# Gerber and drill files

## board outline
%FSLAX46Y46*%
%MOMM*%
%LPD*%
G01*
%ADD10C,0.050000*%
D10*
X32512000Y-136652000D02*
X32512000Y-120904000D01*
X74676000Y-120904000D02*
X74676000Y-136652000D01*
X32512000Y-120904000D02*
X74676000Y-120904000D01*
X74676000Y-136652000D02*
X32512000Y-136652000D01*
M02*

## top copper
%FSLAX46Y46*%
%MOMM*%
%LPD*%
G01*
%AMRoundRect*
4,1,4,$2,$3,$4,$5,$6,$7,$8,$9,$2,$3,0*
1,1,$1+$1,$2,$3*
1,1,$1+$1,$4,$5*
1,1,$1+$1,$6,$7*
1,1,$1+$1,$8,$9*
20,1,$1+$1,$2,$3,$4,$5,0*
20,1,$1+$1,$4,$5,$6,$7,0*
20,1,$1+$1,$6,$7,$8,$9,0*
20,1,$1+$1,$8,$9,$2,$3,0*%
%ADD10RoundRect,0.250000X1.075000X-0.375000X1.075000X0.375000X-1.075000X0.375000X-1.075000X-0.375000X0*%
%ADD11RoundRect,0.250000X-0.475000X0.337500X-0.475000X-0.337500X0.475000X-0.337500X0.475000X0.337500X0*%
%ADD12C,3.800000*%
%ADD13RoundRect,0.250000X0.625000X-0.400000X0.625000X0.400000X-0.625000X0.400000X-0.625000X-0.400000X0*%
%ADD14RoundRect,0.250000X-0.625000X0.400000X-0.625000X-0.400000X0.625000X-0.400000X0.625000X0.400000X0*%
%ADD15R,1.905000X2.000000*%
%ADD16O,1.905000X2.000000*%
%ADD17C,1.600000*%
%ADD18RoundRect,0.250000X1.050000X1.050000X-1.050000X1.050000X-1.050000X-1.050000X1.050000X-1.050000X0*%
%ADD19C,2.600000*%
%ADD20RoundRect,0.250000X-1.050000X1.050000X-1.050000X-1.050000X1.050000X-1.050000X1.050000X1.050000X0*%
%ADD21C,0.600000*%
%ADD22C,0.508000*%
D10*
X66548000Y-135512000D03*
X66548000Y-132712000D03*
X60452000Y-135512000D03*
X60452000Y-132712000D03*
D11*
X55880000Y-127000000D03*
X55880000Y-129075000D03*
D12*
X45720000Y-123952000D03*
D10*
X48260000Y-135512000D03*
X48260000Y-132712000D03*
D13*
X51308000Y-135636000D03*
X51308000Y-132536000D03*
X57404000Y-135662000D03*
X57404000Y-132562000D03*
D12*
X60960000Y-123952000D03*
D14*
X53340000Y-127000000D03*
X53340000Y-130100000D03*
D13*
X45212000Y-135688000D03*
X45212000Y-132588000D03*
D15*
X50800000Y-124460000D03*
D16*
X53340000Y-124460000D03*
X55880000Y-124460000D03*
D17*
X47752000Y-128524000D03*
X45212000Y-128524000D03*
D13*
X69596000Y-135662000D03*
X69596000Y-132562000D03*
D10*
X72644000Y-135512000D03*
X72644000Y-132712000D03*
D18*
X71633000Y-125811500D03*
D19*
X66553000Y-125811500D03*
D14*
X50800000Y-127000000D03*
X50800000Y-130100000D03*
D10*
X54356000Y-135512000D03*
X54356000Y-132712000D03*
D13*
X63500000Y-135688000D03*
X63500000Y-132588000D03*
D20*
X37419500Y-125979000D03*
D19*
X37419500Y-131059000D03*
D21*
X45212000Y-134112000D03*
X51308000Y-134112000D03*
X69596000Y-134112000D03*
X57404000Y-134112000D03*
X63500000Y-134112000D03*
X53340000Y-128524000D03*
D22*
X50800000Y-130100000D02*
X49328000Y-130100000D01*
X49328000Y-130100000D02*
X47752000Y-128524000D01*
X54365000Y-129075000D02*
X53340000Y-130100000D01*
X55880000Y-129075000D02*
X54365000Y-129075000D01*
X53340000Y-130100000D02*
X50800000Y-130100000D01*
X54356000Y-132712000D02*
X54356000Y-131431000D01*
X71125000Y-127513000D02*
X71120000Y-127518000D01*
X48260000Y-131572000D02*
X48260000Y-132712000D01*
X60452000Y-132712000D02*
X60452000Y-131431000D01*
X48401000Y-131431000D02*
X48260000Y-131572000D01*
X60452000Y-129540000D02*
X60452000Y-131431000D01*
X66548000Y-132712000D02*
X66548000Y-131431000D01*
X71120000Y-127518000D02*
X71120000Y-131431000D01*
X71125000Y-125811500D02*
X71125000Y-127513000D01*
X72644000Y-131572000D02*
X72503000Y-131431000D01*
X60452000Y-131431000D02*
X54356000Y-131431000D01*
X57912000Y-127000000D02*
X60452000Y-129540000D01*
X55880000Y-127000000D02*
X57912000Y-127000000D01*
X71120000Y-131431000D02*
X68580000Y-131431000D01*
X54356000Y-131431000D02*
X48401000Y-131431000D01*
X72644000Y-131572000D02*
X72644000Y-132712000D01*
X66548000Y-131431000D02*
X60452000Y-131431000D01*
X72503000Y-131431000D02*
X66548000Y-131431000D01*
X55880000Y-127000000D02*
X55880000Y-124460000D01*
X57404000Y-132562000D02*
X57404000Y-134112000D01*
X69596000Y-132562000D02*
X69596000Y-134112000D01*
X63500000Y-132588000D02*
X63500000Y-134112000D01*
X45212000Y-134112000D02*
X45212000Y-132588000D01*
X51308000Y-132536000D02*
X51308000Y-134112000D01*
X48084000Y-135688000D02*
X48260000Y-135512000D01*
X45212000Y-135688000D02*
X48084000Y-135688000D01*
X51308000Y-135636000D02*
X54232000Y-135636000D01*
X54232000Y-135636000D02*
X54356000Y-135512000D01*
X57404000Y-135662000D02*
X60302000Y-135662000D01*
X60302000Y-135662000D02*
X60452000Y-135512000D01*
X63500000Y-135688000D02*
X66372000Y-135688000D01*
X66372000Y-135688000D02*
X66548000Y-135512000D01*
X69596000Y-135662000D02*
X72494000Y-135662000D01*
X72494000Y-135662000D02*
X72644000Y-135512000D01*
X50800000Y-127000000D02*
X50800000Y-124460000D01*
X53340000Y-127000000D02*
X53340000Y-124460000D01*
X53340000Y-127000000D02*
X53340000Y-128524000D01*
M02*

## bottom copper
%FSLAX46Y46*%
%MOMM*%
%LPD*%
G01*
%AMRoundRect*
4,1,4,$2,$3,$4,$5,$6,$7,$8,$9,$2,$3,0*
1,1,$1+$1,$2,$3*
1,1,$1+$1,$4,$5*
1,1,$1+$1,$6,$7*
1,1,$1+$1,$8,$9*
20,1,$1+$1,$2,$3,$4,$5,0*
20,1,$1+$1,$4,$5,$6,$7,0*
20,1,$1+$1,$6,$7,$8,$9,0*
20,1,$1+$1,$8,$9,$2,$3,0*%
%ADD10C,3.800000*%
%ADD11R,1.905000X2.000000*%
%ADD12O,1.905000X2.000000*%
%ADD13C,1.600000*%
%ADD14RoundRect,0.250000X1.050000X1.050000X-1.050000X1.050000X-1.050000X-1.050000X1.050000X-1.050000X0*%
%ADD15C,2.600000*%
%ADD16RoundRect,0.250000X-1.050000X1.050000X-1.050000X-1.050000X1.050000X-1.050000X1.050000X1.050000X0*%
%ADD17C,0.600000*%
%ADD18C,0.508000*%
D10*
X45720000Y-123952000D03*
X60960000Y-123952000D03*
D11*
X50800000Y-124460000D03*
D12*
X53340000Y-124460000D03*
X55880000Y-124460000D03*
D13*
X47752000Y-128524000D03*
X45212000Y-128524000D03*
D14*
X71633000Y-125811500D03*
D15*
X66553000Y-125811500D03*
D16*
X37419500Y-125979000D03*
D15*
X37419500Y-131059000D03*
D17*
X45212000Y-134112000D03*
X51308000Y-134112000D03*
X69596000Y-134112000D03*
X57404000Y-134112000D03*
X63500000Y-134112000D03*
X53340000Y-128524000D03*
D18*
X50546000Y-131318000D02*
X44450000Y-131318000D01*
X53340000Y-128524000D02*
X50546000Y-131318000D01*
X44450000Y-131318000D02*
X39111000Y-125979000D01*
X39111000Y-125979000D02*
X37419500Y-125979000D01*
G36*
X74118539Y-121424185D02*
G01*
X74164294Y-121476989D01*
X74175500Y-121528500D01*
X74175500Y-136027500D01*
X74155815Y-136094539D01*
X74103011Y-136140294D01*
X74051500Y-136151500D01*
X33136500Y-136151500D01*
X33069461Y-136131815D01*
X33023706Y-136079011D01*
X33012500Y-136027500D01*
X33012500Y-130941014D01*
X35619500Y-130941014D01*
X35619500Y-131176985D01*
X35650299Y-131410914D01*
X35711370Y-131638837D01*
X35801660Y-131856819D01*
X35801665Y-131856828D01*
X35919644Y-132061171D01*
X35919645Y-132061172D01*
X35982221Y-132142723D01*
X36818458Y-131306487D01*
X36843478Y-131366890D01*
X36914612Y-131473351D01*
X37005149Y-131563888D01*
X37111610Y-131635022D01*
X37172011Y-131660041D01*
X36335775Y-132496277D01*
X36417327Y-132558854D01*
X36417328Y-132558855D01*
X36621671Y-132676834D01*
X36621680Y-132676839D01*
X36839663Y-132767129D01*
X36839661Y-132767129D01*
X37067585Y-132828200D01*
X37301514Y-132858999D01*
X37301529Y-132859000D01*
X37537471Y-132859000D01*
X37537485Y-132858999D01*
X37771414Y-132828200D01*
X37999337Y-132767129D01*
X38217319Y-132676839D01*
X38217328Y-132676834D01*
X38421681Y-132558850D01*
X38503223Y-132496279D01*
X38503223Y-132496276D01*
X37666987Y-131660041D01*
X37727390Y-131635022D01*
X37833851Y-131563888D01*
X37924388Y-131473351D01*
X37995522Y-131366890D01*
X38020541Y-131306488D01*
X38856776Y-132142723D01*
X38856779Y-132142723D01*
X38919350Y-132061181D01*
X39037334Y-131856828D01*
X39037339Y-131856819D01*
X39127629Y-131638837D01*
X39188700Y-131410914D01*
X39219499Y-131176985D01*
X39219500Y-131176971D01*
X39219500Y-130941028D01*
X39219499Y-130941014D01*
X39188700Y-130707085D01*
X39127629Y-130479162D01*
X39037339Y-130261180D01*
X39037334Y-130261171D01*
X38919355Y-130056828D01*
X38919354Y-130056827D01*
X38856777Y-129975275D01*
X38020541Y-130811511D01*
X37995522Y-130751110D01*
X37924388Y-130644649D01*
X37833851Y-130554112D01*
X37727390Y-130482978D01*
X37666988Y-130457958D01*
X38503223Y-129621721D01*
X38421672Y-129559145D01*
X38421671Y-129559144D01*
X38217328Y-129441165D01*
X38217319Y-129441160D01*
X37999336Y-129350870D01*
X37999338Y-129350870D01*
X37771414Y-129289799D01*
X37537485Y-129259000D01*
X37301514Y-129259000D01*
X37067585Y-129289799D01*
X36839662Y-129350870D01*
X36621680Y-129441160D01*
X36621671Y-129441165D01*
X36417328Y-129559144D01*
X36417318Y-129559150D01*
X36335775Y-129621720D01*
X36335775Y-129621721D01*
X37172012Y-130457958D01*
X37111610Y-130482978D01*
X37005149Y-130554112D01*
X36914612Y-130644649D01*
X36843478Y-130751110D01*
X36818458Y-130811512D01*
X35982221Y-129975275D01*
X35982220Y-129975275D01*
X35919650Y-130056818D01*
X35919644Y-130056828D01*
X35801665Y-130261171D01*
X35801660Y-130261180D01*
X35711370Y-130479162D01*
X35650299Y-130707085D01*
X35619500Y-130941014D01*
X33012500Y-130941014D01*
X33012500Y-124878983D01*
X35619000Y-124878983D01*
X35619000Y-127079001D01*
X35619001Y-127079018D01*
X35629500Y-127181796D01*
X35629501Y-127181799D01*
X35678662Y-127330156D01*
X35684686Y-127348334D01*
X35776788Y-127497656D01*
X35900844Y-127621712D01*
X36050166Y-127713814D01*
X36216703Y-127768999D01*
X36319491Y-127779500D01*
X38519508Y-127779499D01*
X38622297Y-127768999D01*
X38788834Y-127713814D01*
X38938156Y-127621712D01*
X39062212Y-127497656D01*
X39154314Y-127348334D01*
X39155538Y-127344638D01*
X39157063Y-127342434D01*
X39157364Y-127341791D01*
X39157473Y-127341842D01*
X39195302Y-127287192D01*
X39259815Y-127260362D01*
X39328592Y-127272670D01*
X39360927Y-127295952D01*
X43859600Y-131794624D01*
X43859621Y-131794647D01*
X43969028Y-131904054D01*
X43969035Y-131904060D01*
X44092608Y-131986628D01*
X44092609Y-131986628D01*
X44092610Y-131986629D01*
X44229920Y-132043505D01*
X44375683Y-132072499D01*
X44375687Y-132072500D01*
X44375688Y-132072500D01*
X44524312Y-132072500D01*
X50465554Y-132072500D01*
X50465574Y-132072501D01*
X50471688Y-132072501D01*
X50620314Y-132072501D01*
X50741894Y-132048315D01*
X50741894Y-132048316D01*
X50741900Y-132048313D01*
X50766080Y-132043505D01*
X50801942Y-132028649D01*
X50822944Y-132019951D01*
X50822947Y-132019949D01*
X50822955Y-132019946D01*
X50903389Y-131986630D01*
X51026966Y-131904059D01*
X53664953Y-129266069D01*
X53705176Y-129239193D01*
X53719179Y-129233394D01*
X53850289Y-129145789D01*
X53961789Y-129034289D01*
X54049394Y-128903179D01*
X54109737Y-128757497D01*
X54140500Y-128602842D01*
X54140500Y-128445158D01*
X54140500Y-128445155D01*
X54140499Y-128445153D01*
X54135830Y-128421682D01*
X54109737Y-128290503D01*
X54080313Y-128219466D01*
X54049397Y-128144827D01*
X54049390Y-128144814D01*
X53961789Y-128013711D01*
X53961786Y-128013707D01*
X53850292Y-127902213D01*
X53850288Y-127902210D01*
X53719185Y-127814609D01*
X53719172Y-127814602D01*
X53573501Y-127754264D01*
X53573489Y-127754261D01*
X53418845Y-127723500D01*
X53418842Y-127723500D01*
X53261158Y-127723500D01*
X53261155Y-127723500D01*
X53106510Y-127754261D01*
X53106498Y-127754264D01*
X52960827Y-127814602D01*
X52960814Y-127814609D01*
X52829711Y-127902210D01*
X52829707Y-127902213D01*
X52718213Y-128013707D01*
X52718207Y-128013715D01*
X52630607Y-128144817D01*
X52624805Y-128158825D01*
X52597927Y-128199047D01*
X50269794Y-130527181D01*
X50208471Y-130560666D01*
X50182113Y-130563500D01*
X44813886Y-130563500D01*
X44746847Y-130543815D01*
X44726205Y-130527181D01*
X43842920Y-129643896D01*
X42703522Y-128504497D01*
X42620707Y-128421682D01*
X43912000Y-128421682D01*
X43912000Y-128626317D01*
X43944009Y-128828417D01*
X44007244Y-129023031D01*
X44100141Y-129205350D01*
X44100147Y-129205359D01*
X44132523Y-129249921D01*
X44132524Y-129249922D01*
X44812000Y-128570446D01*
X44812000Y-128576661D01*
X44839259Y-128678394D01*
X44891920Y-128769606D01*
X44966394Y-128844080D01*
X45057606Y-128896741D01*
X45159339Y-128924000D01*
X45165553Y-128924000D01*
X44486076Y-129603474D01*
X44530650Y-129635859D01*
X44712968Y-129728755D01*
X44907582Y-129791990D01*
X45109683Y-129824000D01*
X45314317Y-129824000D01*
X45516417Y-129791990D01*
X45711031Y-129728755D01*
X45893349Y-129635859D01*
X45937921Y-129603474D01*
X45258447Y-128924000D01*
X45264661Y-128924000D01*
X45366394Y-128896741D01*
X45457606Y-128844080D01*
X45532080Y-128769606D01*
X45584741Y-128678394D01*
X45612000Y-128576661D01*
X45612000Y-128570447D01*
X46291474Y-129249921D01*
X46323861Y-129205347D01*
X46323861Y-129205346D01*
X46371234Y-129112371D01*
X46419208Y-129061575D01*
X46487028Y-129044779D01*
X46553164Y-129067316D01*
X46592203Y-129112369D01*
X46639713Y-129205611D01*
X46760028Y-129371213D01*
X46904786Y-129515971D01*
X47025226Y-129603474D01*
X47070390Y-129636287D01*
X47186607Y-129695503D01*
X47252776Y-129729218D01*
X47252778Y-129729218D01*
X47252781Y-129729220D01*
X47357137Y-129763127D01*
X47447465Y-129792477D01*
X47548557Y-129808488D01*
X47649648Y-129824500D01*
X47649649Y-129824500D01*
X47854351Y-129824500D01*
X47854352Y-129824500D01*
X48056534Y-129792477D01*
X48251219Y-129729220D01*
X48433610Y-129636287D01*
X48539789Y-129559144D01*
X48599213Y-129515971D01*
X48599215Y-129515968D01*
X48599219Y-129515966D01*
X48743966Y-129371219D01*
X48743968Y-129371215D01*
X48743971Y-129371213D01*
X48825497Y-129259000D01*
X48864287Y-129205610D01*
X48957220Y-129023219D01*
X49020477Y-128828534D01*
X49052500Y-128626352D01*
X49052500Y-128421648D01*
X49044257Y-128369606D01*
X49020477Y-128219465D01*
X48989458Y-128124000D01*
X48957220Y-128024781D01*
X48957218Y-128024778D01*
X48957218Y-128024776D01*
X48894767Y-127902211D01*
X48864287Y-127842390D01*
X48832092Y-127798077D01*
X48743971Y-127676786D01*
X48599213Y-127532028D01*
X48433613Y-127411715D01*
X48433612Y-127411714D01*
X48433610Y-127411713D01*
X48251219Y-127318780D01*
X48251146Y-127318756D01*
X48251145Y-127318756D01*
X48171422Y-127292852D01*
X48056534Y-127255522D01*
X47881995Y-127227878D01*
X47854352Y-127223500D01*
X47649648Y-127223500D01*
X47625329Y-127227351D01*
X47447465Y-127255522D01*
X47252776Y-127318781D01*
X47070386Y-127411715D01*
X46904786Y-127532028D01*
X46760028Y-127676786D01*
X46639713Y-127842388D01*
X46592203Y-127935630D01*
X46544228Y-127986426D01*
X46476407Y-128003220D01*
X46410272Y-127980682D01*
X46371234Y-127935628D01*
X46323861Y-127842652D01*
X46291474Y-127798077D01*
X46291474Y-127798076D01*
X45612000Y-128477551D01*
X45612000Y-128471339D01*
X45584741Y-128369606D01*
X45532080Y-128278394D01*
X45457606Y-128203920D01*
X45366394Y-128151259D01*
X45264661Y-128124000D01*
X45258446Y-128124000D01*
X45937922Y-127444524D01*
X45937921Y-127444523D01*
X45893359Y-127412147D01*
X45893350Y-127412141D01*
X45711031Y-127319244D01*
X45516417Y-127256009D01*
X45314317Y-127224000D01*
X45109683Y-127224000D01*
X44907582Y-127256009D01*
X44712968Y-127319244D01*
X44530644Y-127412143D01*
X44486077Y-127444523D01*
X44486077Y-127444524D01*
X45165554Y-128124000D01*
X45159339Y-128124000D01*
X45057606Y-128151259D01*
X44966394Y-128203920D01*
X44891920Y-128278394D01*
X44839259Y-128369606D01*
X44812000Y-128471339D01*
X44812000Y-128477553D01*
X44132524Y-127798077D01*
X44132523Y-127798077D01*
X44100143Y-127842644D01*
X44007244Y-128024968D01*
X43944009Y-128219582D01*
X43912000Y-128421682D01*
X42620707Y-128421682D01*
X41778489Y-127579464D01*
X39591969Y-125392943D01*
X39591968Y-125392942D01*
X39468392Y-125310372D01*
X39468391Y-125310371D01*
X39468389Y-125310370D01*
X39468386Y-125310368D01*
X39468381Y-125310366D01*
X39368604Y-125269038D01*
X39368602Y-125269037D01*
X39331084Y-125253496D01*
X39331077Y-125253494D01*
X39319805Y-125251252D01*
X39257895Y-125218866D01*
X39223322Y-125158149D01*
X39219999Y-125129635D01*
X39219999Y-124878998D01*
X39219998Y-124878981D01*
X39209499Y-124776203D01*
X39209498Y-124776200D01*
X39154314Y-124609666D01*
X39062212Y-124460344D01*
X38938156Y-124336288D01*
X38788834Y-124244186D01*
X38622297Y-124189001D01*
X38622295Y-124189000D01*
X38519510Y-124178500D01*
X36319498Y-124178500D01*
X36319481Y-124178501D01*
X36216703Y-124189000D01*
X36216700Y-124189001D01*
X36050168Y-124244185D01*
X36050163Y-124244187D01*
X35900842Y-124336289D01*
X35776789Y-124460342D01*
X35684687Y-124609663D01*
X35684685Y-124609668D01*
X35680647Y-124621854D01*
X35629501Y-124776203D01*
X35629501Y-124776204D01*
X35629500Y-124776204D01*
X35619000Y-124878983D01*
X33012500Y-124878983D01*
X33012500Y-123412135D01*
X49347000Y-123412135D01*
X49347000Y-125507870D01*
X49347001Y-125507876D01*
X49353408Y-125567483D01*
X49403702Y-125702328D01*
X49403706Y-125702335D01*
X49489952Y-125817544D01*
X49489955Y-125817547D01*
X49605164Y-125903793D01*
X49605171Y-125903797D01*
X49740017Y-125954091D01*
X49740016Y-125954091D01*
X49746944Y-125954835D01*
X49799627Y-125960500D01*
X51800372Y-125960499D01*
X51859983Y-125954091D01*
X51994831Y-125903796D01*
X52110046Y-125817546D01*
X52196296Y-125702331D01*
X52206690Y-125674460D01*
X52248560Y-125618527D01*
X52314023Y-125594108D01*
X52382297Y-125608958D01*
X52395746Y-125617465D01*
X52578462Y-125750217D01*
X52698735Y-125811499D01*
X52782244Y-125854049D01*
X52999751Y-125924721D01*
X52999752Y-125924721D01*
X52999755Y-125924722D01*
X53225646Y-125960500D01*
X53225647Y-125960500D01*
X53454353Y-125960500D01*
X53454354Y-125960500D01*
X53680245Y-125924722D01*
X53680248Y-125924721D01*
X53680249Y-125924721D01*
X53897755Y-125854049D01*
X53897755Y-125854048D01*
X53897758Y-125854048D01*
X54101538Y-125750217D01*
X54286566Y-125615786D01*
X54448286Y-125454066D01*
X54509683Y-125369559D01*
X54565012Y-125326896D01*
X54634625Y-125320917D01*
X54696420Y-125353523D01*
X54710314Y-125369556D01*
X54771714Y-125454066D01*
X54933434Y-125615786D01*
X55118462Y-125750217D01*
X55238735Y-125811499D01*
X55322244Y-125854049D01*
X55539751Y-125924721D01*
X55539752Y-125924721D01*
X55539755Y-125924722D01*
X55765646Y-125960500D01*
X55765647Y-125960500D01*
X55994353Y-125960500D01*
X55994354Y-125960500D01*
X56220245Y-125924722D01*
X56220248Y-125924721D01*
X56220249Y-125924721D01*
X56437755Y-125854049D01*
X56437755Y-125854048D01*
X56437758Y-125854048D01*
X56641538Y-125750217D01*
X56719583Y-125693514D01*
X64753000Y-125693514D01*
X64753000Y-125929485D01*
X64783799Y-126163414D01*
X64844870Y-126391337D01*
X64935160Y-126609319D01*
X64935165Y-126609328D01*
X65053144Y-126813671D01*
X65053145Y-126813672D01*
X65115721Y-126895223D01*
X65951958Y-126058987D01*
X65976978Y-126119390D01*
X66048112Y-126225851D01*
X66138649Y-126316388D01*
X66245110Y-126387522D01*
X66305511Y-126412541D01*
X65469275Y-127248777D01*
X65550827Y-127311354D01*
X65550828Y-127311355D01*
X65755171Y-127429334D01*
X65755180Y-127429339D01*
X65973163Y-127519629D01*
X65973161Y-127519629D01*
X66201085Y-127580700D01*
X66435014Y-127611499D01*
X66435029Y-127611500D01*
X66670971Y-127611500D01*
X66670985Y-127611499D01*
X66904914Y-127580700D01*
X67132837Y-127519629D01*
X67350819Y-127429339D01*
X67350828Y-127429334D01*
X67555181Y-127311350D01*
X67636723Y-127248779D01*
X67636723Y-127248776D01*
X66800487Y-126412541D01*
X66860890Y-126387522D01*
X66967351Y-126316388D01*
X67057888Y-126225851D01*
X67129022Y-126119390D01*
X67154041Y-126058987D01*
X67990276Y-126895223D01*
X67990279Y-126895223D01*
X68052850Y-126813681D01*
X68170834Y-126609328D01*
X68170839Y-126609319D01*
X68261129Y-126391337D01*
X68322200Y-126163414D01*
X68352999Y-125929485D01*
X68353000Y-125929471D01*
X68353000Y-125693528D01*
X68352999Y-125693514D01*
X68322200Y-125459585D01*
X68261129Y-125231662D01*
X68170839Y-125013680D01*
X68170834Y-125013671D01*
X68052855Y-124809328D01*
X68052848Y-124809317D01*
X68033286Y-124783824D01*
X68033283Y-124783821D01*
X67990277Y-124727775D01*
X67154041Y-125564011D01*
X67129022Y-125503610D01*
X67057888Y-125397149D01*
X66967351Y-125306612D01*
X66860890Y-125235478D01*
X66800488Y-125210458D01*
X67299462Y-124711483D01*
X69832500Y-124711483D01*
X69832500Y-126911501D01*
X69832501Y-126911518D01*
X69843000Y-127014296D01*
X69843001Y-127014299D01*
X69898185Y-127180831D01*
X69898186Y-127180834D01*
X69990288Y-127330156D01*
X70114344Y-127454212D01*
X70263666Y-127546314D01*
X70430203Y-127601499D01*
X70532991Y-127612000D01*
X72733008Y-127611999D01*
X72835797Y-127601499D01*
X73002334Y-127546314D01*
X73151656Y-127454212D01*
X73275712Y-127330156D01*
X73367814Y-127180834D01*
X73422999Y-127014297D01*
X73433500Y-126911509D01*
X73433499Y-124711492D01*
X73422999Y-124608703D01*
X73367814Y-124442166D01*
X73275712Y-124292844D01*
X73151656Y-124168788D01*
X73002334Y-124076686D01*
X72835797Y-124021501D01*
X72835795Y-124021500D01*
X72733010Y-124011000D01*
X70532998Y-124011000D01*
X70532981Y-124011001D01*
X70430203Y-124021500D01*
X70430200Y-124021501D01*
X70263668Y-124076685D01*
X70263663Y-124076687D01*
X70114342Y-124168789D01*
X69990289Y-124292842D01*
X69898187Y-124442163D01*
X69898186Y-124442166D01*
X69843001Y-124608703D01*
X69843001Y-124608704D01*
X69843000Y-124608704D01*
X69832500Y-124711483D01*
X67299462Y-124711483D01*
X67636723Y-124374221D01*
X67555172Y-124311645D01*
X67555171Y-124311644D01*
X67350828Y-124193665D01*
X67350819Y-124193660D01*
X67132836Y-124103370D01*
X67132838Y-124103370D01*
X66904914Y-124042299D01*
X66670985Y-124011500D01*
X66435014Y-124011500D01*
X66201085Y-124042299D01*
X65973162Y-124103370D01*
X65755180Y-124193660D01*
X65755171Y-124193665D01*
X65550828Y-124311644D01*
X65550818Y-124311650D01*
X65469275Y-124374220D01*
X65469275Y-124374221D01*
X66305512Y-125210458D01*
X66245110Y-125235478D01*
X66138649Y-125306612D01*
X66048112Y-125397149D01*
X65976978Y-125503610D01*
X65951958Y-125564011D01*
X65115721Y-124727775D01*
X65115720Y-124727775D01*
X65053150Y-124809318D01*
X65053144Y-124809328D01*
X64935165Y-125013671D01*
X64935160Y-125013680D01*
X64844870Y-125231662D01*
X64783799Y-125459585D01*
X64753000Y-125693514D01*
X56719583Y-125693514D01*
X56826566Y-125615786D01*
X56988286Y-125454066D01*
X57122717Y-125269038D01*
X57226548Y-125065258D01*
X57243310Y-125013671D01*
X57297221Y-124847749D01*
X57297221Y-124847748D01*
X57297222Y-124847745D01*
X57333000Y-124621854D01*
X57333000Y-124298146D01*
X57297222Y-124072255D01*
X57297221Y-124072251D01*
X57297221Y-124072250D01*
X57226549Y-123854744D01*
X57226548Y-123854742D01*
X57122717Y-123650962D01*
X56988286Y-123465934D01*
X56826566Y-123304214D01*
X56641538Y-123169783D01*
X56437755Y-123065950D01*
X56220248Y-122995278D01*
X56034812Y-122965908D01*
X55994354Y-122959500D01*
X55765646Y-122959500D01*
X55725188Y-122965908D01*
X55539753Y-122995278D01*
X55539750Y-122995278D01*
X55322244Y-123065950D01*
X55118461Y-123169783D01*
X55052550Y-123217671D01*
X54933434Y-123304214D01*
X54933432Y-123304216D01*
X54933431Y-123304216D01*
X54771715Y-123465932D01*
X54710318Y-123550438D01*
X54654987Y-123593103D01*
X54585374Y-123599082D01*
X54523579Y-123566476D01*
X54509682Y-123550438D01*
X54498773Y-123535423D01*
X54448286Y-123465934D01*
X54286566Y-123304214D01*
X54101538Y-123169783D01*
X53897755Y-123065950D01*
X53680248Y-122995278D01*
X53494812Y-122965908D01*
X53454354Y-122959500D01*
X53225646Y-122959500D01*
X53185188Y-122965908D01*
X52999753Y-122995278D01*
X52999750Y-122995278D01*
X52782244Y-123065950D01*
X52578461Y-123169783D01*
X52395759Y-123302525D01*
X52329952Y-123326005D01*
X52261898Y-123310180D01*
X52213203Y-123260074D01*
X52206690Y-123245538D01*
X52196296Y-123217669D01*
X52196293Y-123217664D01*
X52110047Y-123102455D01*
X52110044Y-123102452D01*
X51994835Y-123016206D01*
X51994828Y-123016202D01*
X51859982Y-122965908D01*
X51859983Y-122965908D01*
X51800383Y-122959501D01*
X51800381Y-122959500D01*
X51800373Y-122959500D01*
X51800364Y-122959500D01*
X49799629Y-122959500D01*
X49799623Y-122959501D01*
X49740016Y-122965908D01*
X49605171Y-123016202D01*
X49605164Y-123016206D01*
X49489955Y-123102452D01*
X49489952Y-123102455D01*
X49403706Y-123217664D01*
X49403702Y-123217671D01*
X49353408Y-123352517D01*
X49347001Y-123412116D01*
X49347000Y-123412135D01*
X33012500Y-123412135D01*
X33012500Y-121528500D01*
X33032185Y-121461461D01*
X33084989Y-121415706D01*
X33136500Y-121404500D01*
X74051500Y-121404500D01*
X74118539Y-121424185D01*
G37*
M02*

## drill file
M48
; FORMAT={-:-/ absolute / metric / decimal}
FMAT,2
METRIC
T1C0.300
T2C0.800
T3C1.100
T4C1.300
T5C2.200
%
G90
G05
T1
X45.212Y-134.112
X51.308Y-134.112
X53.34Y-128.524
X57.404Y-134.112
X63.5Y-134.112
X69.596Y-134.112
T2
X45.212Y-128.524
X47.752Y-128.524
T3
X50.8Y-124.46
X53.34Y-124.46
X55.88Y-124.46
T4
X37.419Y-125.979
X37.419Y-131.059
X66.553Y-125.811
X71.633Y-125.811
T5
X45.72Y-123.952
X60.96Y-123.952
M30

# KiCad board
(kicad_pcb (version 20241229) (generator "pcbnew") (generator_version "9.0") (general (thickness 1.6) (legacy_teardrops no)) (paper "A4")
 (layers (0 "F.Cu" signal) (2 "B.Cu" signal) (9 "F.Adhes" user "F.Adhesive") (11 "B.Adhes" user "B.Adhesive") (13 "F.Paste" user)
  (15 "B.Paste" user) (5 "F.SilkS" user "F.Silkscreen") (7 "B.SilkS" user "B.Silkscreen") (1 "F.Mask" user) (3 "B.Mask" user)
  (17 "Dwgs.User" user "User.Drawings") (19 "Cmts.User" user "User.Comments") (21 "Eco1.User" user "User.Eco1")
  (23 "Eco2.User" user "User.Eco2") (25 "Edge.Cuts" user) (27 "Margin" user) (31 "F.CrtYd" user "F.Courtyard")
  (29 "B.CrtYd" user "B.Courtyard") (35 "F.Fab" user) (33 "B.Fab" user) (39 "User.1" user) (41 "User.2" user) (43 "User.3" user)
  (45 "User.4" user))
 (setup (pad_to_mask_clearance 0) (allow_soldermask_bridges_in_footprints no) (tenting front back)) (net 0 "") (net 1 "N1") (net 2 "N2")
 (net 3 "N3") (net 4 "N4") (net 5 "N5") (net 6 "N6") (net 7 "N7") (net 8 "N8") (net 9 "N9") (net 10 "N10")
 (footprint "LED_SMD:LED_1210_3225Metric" (layer "F.Cu") (at 66.548 134.112 90)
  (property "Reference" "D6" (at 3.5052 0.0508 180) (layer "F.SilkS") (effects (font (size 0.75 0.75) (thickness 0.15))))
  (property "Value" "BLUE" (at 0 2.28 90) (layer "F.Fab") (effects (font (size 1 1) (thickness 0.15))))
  (pad "1" smd roundrect (at -1.4 0 90) (size 1.25 2.65) (layers "F.Cu" "F.Mask" "F.Paste") (roundrect_rratio 0.2) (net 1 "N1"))
  (pad "2" smd roundrect (at 1.4 0 90) (size 1.25 2.65) (layers "F.Cu" "F.Mask" "F.Paste") (roundrect_rratio 0.2) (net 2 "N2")))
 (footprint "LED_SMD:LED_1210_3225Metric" (layer "F.Cu") (at 60.452 134.112 90)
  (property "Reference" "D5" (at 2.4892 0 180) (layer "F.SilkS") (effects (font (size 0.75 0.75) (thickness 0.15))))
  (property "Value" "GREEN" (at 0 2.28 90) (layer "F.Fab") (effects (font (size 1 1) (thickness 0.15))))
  (pad "1" smd roundrect (at -1.4 0 90) (size 1.25 2.65) (layers "F.Cu" "F.Mask" "F.Paste") (roundrect_rratio 0.2) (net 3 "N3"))
  (pad "2" smd roundrect (at 1.4 0 90) (size 1.25 2.65) (layers "F.Cu" "F.Mask" "F.Paste") (roundrect_rratio 0.2) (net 2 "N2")))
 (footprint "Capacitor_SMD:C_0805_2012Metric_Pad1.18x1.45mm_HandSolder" (layer "F.Cu") (at 55.88 128.0375 -90)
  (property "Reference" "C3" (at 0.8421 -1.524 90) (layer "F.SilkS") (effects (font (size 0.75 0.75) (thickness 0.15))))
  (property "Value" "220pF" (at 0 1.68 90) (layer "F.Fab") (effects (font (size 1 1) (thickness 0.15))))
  (pad "1" smd roundrect (at -1.0375 0 270) (size 1.175 1.45) (layers "F.Cu" "F.Mask" "F.Paste") (roundrect_rratio 0.212766) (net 2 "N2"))
  (pad "2" smd roundrect (at 1.0375 0 270) (size 1.175 1.45) (layers "F.Cu" "F.Mask" "F.Paste") (roundrect_rratio 0.212766) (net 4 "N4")))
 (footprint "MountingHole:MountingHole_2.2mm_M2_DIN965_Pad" (layer "F.Cu") (at 45.72 123.952)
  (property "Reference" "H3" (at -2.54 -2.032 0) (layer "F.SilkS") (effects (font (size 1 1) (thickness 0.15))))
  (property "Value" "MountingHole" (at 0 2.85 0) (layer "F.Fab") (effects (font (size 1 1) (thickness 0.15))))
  (pad "1" thru_hole circle (at 0 0) (size 3.8 3.8) (drill 2.2) (layers "*.Cu" "*.Mask") (remove_unused_layers no) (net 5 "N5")
   (zone_connect 2)))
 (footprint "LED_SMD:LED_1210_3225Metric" (layer "F.Cu") (at 48.26 134.112 90)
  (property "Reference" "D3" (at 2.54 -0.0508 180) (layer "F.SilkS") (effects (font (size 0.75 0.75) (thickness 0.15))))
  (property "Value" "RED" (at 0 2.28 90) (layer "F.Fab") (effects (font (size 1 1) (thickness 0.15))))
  (pad "1" smd roundrect (at -1.4 0 90) (size 1.25 2.65) (layers "F.Cu" "F.Mask" "F.Paste") (roundrect_rratio 0.2) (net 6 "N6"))
  (pad "2" smd roundrect (at 1.4 0 90) (size 1.25 2.65) (layers "F.Cu" "F.Mask" "F.Paste") (roundrect_rratio 0.2) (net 2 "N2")))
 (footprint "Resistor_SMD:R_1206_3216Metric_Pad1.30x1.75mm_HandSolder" (layer "F.Cu") (at 51.308 134.086 90)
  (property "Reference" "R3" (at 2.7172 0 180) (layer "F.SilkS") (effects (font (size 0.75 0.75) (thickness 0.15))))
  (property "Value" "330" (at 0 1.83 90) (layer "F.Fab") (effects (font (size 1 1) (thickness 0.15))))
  (pad "1" smd roundrect (at -1.55 0 90) (size 1.3 1.75) (layers "F.Cu" "F.Mask" "F.Paste") (roundrect_rratio 0.192308) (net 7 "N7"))
  (pad "2" smd roundrect (at 1.55 0 90) (size 1.3 1.75) (layers "F.Cu" "F.Mask" "F.Paste") (roundrect_rratio 0.192308) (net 5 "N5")))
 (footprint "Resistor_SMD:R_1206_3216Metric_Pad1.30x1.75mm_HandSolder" (layer "F.Cu") (at 57.404 134.112 90)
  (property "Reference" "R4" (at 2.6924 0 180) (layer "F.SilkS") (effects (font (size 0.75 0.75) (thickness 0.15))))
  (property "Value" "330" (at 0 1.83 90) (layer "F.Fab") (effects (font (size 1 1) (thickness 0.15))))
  (pad "1" smd roundrect (at -1.55 0 90) (size 1.3 1.75) (layers "F.Cu" "F.Mask" "F.Paste") (roundrect_rratio 0.192308) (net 3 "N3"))
  (pad "2" smd roundrect (at 1.55 0 90) (size 1.3 1.75) (layers "F.Cu" "F.Mask" "F.Paste") (roundrect_rratio 0.192308) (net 5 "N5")))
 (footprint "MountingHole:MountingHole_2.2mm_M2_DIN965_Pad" (layer "F.Cu") (at 60.96 123.952)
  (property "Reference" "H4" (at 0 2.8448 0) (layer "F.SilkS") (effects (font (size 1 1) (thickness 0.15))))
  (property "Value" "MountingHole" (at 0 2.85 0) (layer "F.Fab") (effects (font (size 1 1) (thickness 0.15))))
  (pad "1" thru_hole circle (at 0 0) (size 3.8 3.8) (drill 2.2) (layers "*.Cu" "*.Mask") (remove_unused_layers no) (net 5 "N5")
   (zone_connect 2)))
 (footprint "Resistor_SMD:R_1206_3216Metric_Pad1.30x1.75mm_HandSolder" (layer "F.Cu") (at 53.34 128.55 -90)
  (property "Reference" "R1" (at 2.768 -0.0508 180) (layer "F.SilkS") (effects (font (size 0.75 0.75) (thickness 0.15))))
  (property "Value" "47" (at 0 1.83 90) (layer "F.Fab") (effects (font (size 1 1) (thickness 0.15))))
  (pad "1" smd roundrect (at -1.55 0 270) (size 1.3 1.75) (layers "F.Cu" "F.Mask" "F.Paste") (roundrect_rratio 0.192308) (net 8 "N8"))
  (pad "2" smd roundrect (at 1.55 0 270) (size 1.3 1.75) (layers "F.Cu" "F.Mask" "F.Paste") (roundrect_rratio 0.192308) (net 4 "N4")))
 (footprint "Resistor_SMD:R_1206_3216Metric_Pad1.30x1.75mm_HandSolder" (layer "F.Cu") (at 45.212 134.138 90)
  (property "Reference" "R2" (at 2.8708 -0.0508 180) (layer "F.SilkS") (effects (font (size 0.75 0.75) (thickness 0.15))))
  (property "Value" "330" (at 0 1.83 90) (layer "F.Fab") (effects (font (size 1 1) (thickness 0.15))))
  (pad "1" smd roundrect (at -1.55 0 90) (size 1.3 1.75) (layers "F.Cu" "F.Mask" "F.Paste") (roundrect_rratio 0.192308) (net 6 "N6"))
  (pad "2" smd roundrect (at 1.55 0 90) (size 1.3 1.75) (layers "F.Cu" "F.Mask" "F.Paste") (roundrect_rratio 0.192308) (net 5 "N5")))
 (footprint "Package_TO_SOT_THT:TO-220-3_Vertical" (layer "F.Cu") (at 50.8 124.46)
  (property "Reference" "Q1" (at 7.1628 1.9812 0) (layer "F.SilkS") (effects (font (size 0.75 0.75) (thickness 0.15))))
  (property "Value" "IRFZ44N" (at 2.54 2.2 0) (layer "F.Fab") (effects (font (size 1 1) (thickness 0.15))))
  (pad "1" thru_hole rect (at 0 0) (size 1.905 2) (drill 1.1) (layers "*.Cu" "*.Mask") (remove_unused_layers no) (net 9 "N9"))
  (pad "2" thru_hole oval (at 2.54 0) (size 1.905 2) (drill 1.1) (layers "*.Cu" "*.Mask") (remove_unused_layers no) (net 8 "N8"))
  (pad "3" thru_hole oval (at 5.08 0) (size 1.905 2) (drill 1.1) (layers "*.Cu" "*.Mask") (remove_unused_layers no) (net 2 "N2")))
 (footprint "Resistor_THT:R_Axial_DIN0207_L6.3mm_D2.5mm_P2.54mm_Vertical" (layer "F.Cu") (at 47.752 128.524 180)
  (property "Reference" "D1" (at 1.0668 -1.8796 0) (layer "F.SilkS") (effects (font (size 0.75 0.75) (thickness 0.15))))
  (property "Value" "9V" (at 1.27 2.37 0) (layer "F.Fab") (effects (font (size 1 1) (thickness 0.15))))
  (pad "1" thru_hole circle (at 0 0 180) (size 1.6 1.6) (drill 0.8) (layers "*.Cu" "*.Mask") (remove_unused_layers no) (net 4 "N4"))
  (pad "2" thru_hole circle (at 2.54 0 180) (size 1.6 1.6) (drill 0.8) (layers "*.Cu" "*.Mask") (remove_unused_layers no) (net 5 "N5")))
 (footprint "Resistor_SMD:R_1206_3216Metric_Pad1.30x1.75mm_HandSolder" (layer "F.Cu") (at 69.596 134.112 90)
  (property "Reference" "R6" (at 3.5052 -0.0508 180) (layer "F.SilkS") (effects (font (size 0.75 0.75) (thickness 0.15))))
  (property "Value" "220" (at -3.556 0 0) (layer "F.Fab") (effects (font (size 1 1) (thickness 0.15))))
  (pad "1" smd roundrect (at -1.55 0 90) (size 1.3 1.75) (layers "F.Cu" "F.Mask" "F.Paste") (roundrect_rratio 0.192308) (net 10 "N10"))
  (pad "2" smd roundrect (at 1.55 0 90) (size 1.3 1.75) (layers "F.Cu" "F.Mask" "F.Paste") (roundrect_rratio 0.192308) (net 5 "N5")))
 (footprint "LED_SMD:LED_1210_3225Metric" (layer "F.Cu") (at 72.644 134.112 90)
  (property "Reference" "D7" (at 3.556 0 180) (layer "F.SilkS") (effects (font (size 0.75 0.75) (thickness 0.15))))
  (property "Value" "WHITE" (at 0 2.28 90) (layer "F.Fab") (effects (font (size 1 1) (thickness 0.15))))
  (pad "1" smd roundrect (at -1.4 0 90) (size 1.25 2.65) (layers "F.Cu" "F.Mask" "F.Paste") (roundrect_rratio 0.2) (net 10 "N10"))
  (pad "2" smd roundrect (at 1.4 0 90) (size 1.25 2.65) (layers "F.Cu" "F.Mask" "F.Paste") (roundrect_rratio 0.2) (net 2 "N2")))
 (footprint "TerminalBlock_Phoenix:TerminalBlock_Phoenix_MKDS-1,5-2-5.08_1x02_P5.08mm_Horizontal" (layer "F.Cu") (at 71.633 125.8115 180)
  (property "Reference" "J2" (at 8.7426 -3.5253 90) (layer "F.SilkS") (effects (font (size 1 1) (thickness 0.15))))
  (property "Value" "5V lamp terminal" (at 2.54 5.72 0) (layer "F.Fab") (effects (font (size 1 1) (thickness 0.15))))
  (pad "1" thru_hole roundrect (at 0 0 180) (size 2.6 2.6) (drill 1.3) (layers "*.Cu" "*.Mask") (remove_unused_layers no)
   (roundrect_rratio 0.096154) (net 2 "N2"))
  (pad "2" thru_hole circle (at 5.08 0 180) (size 2.6 2.6) (drill 1.3) (layers "*.Cu" "*.Mask") (remove_unused_layers no) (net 5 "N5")))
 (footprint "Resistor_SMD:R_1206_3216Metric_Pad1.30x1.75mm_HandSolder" (layer "F.Cu") (at 50.8 128.55 -90)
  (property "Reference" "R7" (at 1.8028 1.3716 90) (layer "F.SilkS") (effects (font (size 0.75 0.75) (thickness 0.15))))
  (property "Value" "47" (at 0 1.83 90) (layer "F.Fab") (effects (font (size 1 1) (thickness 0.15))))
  (pad "1" smd roundrect (at -1.55 0 270) (size 1.3 1.75) (layers "F.Cu" "F.Mask" "F.Paste") (roundrect_rratio 0.192308) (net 9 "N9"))
  (pad "2" smd roundrect (at 1.55 0 270) (size 1.3 1.75) (layers "F.Cu" "F.Mask" "F.Paste") (roundrect_rratio 0.192308) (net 4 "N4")))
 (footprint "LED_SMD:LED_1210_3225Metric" (layer "F.Cu") (at 54.356 134.112 90)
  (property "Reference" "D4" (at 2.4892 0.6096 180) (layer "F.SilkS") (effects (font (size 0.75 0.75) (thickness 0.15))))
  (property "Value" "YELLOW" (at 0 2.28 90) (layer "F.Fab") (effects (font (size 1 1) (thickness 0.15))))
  (pad "1" smd roundrect (at -1.4 0 90) (size 1.25 2.65) (layers "F.Cu" "F.Mask" "F.Paste") (roundrect_rratio 0.2) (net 7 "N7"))
  (pad "2" smd roundrect (at 1.4 0 90) (size 1.25 2.65) (layers "F.Cu" "F.Mask" "F.Paste") (roundrect_rratio 0.2) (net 2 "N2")))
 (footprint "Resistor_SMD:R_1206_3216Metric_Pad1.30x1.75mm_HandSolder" (layer "F.Cu") (at 63.5 134.138 90)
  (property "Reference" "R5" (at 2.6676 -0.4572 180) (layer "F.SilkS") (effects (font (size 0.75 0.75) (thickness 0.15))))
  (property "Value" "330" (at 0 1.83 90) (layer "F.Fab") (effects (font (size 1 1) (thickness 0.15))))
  (pad "1" smd roundrect (at -1.55 0 90) (size 1.3 1.75) (layers "F.Cu" "F.Mask" "F.Paste") (roundrect_rratio 0.192308) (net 1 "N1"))
  (pad "2" smd roundrect (at 1.55 0 90) (size 1.3 1.75) (layers "F.Cu" "F.Mask" "F.Paste") (roundrect_rratio 0.192308) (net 5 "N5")))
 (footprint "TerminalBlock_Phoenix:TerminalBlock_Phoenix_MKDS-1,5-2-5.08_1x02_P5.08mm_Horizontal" (layer "F.Cu") (at 37.4195 125.979 -90)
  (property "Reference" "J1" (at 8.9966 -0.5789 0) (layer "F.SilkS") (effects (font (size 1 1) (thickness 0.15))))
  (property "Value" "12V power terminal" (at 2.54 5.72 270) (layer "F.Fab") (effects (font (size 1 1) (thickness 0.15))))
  (pad "1" thru_hole roundrect (at 0 0 270) (size 2.6 2.6) (drill 1.3) (layers "*.Cu" "*.Mask") (remove_unused_layers no)
   (roundrect_rratio 0.096154) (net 8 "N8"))
  (pad "2" thru_hole circle (at 5.08 0 270) (size 2.6 2.6) (drill 1.3) (layers "*.Cu" "*.Mask") (remove_unused_layers no) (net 5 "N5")))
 (gr_line (start 32.512 136.652) (end 32.512 120.904) (stroke (width 0.05) (type default)) (layer "Edge.Cuts"))
 (gr_line (start 74.676 120.904) (end 74.676 136.652) (stroke (width 0.05) (type default)) (layer "Edge.Cuts"))
 (gr_line (start 32.512 120.904) (end 74.676 120.904) (stroke (width 0.05) (type default)) (layer "Edge.Cuts"))
 (gr_line (start 74.676 136.652) (end 32.512 136.652) (stroke (width 0.05) (type default)) (layer "Edge.Cuts"))
 (segment (start 50.8 130.1) (end 49.328 130.1) (width 0.508) (layer "F.Cu") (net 4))
 (segment (start 49.328 130.1) (end 47.752 128.524) (width 0.508) (layer "F.Cu") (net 4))
 (segment (start 54.365 129.075) (end 53.34 130.1) (width 0.508) (layer "F.Cu") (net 4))
 (segment (start 55.88 129.075) (end 54.365 129.075) (width 0.508) (layer "F.Cu") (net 4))
 (segment (start 53.34 130.1) (end 50.8 130.1) (width 0.508) (layer "F.Cu") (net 4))
 (segment (start 54.356 132.712) (end 54.356 131.431) (width 0.508) (layer "F.Cu") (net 2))
 (segment (start 71.125 127.513) (end 71.12 127.518) (width 0.508) (layer "F.Cu") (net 2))
 (segment (start 48.26 131.572) (end 48.26 132.712) (width 0.508) (layer "F.Cu") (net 2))
 (segment (start 60.452 132.712) (end 60.452 131.431) (width 0.508) (layer "F.Cu") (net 2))
 (segment (start 48.401 131.431) (end 48.26 131.572) (width 0.508) (layer "F.Cu") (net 2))
 (segment (start 60.452 129.54) (end 60.452 131.431) (width 0.508) (layer "F.Cu") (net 2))
 (segment (start 66.548 132.712) (end 66.548 131.431) (width 0.508) (layer "F.Cu") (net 2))
 (segment (start 71.12 127.518) (end 71.12 131.431) (width 0.508) (layer "F.Cu") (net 2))
 (segment (start 71.125 125.8115) (end 71.125 127.513) (width 0.508) (layer "F.Cu") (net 2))
 (segment (start 72.644 131.572) (end 72.503 131.431) (width 0.508) (layer "F.Cu") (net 2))
 (segment (start 60.452 131.431) (end 54.356 131.431) (width 0.508) (layer "F.Cu") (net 2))
 (segment (start 57.912 127) (end 60.452 129.54) (width 0.508) (layer "F.Cu") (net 2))
 (segment (start 55.88 127) (end 57.912 127) (width 0.508) (layer "F.Cu") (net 2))
 (segment (start 71.12 131.431) (end 68.58 131.431) (width 0.508) (layer "F.Cu") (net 2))
 (segment (start 54.356 131.431) (end 48.401 131.431) (width 0.508) (layer "F.Cu") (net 2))
 (segment (start 72.644 131.572) (end 72.644 132.712) (width 0.508) (layer "F.Cu") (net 2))
 (segment (start 66.548 131.431) (end 60.452 131.431) (width 0.508) (layer "F.Cu") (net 2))
 (segment (start 72.503 131.431) (end 66.548 131.431) (width 0.508) (layer "F.Cu") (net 2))
 (segment (start 55.88 127) (end 55.88 124.46) (width 0.508) (layer "F.Cu") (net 2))
 (segment (start 57.404 132.562) (end 57.404 134.112) (width 0.508) (layer "F.Cu") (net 5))
 (segment (start 69.596 132.562) (end 69.596 134.112) (width 0.508) (layer "F.Cu") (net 5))
 (segment (start 63.5 132.588) (end 63.5 134.112) (width 0.508) (layer "F.Cu") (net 5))
 (segment (start 45.212 134.112) (end 45.212 132.588) (width 0.508) (layer "F.Cu") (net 5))
 (segment (start 51.308 132.536) (end 51.308 134.112) (width 0.508) (layer "F.Cu") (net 5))
 (via (at 45.212 134.112) (size 0.6) (drill 0.3) (layers "F.Cu" "B.Cu") (free yes) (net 5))
 (via (at 51.308 134.112) (size 0.6) (drill 0.3) (layers "F.Cu" "B.Cu") (free yes) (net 5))
 (via (at 69.596 134.112) (size 0.6) (drill 0.3) (layers "F.Cu" "B.Cu") (free yes) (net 5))
 (via (at 57.404 134.112) (size 0.6) (drill 0.3) (layers "F.Cu" "B.Cu") (free yes) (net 5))
 (via (at 63.5 134.112) (size 0.6) (drill 0.3) (layers "F.Cu" "B.Cu") (free yes) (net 5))
 (segment (start 48.084 135.688) (end 48.26 135.512) (width 0.508) (layer "F.Cu") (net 6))
 (segment (start 45.212 135.688) (end 48.084 135.688) (width 0.508) (layer "F.Cu") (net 6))
 (segment (start 51.308 135.636) (end 54.232 135.636) (width 0.508) (layer "F.Cu") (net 7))
 (segment (start 54.232 135.636) (end 54.356 135.512) (width 0.508) (layer "F.Cu") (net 7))
 (segment (start 57.404 135.662) (end 60.302 135.662) (width 0.508) (layer "F.Cu") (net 3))
 (segment (start 60.302 135.662) (end 60.452 135.512) (width 0.508) (layer "F.Cu") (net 3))
 (segment (start 63.5 135.688) (end 66.372 135.688) (width 0.508) (layer "F.Cu") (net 1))
 (segment (start 66.372 135.688) (end 66.548 135.512) (width 0.508) (layer "F.Cu") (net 1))
 (segment (start 69.596 135.662) (end 72.494 135.662) (width 0.508) (layer "F.Cu") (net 10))
 (segment (start 72.494 135.662) (end 72.644 135.512) (width 0.508) (layer "F.Cu") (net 10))
 (segment (start 50.8 127) (end 50.8 124.46) (width 0.508) (layer "F.Cu") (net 9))
 (segment (start 53.34 127) (end 53.34 124.46) (width 0.508) (layer "F.Cu") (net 8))
 (segment (start 53.34 127) (end 53.34 128.524) (width 0.508) (layer "F.Cu") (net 8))
 (via (at 53.34 128.524) (size 0.6) (drill 0.3) (layers "F.Cu" "B.Cu") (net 8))
 (segment (start 50.546 131.318) (end 44.45 131.318) (width 0.508) (layer "B.Cu") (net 8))
 (segment (start 53.34 128.524) (end 50.546 131.318) (width 0.508) (layer "B.Cu") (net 8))
 (segment (start 44.45 131.318) (end 39.111 125.979) (width 0.508) (layer "B.Cu") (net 8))
 (segment (start 39.111 125.979) (end 37.4195 125.979) (width 0.508) (layer "B.Cu") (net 8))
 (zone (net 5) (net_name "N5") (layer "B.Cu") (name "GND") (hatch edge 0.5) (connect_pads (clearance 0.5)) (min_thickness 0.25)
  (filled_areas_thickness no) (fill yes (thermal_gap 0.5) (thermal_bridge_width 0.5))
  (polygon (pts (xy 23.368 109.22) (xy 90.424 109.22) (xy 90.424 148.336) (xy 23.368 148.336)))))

